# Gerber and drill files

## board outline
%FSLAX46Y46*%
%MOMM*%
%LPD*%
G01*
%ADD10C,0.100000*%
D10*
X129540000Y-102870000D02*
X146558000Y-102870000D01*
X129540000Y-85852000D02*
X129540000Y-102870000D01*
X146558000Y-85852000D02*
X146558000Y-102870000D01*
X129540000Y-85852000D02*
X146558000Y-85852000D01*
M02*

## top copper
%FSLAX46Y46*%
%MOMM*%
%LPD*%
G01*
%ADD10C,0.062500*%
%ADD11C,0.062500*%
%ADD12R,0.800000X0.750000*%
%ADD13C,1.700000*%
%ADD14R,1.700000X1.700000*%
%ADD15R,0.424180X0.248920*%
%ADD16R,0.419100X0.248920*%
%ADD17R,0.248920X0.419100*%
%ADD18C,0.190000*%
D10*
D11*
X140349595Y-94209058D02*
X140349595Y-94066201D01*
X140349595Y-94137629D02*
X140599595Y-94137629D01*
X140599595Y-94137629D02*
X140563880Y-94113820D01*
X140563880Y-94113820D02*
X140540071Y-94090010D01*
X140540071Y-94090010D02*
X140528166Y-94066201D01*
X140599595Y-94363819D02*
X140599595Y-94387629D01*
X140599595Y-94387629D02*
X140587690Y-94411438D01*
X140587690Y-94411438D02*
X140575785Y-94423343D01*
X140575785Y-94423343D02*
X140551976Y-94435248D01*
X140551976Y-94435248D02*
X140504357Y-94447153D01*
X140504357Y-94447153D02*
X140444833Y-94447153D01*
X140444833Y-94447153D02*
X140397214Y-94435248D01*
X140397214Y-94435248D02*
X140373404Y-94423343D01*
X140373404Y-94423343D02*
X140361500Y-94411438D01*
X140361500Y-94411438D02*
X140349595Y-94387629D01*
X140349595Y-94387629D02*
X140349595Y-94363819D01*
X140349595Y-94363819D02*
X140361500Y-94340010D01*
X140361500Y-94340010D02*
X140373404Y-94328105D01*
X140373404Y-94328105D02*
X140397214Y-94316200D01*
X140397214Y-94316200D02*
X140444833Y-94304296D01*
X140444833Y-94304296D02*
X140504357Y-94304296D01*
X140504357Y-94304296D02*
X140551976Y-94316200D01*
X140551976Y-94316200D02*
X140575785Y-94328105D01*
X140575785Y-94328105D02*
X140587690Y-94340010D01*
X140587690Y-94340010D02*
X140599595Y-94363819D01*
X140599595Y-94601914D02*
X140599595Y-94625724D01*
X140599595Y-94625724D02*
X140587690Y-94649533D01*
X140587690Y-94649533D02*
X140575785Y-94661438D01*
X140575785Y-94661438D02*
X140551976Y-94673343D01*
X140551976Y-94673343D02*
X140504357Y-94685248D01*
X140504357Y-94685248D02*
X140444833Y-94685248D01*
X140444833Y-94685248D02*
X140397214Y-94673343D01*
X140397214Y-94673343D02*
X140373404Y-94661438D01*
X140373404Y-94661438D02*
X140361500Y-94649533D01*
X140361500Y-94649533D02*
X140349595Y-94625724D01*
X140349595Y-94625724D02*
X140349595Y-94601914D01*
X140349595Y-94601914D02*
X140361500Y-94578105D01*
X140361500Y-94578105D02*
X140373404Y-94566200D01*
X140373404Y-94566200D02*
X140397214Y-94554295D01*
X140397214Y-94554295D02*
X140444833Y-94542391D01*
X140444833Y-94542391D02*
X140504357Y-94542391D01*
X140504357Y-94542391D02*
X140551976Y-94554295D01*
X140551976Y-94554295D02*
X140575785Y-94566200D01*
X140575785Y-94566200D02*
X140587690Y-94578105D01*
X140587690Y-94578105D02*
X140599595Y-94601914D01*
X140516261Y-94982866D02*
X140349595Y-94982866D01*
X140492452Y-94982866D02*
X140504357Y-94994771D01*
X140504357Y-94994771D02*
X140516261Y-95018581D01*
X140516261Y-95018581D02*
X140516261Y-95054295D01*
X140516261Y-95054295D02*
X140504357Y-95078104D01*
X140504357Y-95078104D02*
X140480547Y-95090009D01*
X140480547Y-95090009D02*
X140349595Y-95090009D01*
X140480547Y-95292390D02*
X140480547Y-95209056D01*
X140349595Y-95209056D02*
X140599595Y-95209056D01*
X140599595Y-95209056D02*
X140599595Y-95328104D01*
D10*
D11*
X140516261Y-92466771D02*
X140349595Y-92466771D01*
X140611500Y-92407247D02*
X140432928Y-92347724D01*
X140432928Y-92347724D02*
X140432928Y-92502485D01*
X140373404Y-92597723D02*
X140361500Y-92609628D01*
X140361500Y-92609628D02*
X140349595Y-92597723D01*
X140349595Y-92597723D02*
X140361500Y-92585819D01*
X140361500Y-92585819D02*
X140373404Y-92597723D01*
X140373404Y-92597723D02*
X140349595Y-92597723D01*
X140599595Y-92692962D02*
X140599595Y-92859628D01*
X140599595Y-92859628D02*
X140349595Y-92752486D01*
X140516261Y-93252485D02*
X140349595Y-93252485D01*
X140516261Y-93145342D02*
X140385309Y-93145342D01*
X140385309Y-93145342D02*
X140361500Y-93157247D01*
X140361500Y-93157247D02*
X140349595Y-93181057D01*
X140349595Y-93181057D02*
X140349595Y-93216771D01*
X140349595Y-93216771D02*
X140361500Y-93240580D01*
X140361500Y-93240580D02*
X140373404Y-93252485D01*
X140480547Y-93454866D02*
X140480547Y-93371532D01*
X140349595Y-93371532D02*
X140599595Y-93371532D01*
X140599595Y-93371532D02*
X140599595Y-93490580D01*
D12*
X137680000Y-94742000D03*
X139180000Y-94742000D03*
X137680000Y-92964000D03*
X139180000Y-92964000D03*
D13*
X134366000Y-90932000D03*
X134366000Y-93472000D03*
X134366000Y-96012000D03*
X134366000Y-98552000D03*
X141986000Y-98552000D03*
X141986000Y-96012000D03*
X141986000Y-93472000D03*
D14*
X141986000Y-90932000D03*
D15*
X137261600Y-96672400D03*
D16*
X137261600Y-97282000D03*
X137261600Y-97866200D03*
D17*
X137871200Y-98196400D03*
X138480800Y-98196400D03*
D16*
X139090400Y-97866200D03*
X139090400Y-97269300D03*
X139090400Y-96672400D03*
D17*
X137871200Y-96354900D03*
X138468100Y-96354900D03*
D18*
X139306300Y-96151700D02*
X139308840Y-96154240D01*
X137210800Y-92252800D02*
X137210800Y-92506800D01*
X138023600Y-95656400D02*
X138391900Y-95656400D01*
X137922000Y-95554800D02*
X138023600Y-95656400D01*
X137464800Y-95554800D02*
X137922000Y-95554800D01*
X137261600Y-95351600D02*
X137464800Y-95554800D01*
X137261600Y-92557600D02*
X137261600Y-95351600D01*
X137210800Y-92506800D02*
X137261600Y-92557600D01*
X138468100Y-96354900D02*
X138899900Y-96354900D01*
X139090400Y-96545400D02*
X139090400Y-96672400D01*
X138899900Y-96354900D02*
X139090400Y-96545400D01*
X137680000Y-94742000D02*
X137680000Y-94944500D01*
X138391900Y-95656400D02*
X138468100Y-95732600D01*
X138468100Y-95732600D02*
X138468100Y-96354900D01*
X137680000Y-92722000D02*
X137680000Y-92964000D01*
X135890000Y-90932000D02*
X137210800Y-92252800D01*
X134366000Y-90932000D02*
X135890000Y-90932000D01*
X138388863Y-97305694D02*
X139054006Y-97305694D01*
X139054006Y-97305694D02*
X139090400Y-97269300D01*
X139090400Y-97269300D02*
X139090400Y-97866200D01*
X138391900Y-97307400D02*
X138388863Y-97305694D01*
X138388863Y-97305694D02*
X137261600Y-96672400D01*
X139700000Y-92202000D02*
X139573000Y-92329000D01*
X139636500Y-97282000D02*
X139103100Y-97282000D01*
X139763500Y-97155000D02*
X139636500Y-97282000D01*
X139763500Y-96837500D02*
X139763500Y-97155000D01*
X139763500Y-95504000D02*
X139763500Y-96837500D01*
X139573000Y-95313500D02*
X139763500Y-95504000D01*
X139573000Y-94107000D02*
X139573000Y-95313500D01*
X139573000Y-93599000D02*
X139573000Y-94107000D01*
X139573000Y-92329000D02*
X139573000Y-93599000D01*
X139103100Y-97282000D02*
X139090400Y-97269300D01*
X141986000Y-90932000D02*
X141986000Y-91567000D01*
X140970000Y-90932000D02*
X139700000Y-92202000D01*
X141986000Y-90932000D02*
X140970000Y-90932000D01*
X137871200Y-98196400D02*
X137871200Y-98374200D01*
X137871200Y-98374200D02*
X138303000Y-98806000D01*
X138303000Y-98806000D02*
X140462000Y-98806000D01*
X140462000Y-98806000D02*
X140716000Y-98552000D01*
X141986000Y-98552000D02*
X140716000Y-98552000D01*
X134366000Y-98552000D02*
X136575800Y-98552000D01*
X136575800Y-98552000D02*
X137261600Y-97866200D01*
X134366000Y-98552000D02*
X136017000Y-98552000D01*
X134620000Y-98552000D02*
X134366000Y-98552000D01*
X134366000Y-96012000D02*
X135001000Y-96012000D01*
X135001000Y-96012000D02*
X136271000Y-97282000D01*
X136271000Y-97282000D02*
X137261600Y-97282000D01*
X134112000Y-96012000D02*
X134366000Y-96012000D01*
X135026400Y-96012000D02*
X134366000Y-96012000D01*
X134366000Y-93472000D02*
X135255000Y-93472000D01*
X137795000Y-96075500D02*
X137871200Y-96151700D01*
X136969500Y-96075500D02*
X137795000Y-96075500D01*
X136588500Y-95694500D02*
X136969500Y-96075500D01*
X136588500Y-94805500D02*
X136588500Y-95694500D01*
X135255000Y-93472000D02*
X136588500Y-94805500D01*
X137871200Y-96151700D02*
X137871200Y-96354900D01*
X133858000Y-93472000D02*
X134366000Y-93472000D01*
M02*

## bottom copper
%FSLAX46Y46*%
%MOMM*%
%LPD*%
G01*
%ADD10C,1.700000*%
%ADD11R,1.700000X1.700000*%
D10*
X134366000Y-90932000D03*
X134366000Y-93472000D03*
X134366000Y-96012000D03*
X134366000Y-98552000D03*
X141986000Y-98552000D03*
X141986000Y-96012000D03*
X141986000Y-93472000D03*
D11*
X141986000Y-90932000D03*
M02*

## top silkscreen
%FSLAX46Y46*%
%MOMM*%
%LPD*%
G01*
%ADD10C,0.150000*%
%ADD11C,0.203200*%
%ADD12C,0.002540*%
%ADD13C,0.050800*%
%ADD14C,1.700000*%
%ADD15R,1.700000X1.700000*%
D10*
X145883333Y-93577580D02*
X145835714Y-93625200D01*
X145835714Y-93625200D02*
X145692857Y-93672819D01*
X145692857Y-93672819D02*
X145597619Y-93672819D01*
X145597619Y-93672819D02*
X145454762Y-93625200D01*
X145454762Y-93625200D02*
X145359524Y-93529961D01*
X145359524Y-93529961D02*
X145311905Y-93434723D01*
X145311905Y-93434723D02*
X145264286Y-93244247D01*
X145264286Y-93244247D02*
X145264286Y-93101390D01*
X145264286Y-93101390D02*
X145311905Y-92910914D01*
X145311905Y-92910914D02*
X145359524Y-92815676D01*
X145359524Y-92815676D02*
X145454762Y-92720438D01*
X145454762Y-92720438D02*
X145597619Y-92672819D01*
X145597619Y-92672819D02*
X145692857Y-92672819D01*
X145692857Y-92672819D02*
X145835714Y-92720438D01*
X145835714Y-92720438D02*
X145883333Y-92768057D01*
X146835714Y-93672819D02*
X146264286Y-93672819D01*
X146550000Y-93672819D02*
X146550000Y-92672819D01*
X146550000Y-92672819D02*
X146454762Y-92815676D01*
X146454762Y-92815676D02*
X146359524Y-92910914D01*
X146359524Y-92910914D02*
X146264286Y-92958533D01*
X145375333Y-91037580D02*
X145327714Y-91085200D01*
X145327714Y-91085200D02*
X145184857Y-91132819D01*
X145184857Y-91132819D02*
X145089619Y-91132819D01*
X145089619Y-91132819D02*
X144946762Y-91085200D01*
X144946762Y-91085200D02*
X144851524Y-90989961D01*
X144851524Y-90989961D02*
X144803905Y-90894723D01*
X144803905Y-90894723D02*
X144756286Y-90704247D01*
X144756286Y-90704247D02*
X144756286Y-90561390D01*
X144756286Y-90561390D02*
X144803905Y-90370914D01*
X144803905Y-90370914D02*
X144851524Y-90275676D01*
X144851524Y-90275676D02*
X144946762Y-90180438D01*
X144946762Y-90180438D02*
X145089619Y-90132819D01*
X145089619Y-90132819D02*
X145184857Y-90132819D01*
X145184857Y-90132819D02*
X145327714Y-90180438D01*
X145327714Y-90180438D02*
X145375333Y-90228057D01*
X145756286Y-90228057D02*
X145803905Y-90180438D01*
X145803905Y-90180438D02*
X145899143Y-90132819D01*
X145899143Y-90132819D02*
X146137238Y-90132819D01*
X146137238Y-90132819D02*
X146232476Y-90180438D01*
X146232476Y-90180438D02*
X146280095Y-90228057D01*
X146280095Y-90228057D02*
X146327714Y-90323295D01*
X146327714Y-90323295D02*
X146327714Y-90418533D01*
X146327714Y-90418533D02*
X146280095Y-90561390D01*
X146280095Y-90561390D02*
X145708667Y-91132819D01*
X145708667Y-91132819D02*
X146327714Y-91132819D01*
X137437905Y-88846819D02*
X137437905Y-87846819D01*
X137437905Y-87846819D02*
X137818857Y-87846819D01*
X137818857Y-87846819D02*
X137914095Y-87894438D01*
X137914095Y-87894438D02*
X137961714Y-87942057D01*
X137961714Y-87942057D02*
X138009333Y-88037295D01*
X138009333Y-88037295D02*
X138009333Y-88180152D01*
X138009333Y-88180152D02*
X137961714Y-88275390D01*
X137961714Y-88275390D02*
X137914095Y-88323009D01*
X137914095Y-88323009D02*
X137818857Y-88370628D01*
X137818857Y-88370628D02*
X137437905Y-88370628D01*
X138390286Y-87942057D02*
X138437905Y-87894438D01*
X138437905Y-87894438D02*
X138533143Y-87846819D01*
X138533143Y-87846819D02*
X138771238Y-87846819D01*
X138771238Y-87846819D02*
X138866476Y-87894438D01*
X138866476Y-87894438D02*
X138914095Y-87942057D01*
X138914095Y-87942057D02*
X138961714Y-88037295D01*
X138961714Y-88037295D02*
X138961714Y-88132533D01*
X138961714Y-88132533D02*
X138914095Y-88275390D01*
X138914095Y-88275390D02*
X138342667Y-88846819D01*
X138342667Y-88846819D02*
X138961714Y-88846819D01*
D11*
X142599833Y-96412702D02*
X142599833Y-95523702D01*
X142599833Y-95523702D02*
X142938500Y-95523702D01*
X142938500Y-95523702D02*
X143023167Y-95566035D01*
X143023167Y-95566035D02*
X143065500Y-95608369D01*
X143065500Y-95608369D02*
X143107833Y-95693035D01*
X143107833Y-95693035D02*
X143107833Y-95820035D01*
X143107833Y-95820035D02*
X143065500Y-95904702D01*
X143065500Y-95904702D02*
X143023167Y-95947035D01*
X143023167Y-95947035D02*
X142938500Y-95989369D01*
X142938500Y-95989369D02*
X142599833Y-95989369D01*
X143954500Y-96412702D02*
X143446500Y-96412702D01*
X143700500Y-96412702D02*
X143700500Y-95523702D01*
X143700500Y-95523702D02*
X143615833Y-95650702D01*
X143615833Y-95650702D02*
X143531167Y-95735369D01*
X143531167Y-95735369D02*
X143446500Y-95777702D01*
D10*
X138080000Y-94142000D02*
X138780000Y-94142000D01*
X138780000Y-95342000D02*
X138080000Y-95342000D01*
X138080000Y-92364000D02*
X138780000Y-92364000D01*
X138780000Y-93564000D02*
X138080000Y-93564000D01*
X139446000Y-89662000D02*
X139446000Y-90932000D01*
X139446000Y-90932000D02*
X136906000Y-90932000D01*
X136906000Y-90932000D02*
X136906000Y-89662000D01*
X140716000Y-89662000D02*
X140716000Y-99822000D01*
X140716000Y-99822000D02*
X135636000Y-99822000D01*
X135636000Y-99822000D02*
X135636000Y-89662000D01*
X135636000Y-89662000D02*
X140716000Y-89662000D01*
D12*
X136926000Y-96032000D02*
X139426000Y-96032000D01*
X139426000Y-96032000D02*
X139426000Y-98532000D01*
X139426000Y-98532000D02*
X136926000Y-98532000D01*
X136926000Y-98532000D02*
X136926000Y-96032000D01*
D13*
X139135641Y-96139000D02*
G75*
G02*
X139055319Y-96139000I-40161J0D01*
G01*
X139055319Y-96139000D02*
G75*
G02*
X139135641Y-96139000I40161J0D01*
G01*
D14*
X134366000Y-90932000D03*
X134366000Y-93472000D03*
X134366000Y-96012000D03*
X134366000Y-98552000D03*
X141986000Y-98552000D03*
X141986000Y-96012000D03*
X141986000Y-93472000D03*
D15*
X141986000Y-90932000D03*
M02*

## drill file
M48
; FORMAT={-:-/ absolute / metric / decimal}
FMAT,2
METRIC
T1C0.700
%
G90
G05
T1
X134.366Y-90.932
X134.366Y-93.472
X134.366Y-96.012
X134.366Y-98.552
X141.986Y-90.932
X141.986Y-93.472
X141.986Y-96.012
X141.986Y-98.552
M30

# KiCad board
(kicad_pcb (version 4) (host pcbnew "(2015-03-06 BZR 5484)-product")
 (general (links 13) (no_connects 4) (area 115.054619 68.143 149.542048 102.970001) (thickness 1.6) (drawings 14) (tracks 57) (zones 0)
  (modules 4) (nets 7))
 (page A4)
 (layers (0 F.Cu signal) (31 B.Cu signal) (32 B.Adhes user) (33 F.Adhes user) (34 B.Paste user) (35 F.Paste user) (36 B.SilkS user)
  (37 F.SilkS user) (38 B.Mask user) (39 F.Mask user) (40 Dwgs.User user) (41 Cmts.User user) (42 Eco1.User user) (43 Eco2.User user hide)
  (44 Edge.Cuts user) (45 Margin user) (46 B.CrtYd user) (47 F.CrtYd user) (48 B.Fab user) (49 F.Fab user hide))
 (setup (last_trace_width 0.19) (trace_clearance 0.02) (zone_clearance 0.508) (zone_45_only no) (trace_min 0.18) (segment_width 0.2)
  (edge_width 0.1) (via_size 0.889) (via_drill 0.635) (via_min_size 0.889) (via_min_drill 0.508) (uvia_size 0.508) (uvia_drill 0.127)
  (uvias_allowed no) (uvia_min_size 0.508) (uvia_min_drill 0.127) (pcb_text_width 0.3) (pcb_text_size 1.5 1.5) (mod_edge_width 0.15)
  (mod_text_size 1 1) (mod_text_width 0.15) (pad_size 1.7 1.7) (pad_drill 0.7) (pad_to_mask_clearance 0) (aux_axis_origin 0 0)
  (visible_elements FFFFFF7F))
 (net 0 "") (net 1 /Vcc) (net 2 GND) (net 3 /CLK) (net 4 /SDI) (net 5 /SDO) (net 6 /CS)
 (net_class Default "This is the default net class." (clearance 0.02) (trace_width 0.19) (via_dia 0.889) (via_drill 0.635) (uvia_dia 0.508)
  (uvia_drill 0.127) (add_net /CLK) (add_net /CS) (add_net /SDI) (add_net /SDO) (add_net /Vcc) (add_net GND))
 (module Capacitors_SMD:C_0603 (layer F.Cu) (at 138.43 94.742)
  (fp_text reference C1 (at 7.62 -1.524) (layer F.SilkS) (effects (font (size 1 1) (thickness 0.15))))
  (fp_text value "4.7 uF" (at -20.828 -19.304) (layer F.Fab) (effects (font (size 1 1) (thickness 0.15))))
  (fp_line (start -0.35 -0.6) (end 0.35 -0.6) (layer F.SilkS) (width 0.15))
  (fp_line (start 0.35 0.6) (end -0.35 0.6) (layer F.SilkS) (width 0.15))
  (pad 1 smd rect (at -0.75 0) (size 0.8 0.75) (layers F.Cu F.Paste F.Mask) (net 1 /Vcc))
  (pad 2 smd rect (at 0.75 0) (size 0.8 0.75) (layers F.Cu F.Paste F.Mask) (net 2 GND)))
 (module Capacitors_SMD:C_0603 (layer F.Cu) (at 138.43 92.964)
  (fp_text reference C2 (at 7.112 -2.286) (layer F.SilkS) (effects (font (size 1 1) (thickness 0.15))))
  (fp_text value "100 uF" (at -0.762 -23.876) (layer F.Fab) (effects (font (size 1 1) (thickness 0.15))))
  (fp_line (start -0.35 -0.6) (end 0.35 -0.6) (layer F.SilkS) (width 0.15))
  (fp_line (start 0.35 0.6) (end -0.35 0.6) (layer F.SilkS) (width 0.15))
  (pad 1 smd rect (at -0.75 0) (size 0.8 0.75) (layers F.Cu F.Paste F.Mask) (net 1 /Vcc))
  (pad 2 smd rect (at 0.75 0) (size 0.8 0.75) (layers F.Cu F.Paste F.Mask) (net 2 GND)))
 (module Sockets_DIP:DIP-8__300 (layer F.Cu) (at 138.176 94.742 270)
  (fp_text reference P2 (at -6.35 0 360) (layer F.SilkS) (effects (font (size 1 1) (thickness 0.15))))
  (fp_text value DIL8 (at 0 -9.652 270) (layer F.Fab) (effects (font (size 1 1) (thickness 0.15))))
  (fp_line (start -5.08 -1.27) (end -3.81 -1.27) (layer F.SilkS) (width 0.15))
  (fp_line (start -3.81 -1.27) (end -3.81 1.27) (layer F.SilkS) (width 0.15))
  (fp_line (start -3.81 1.27) (end -5.08 1.27) (layer F.SilkS) (width 0.15))
  (fp_line (start -5.08 -2.54) (end 5.08 -2.54) (layer F.SilkS) (width 0.15))
  (fp_line (start 5.08 -2.54) (end 5.08 2.54) (layer F.SilkS) (width 0.15))
  (fp_line (start 5.08 2.54) (end -5.08 2.54) (layer F.SilkS) (width 0.15))
  (fp_line (start -5.08 2.54) (end -5.08 -2.54) (layer F.SilkS) (width 0.15))
  (pad 1 thru_hole circle (at -3.81 3.81 270) (size 1.7 1.7) (drill 0.7) (layers *.Cu *.Mask F.SilkS) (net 1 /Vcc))
  (pad 2 thru_hole circle (at -1.27 3.81 270) (size 1.7 1.7) (drill 0.7) (layers *.Cu *.Mask F.SilkS) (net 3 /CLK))
  (pad 3 thru_hole circle (at 1.27 3.81 270) (size 1.7 1.7) (drill 0.7) (layers *.Cu *.Mask F.SilkS) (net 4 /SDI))
  (pad 4 thru_hole circle (at 3.81 3.81 270) (size 1.7 1.7) (drill 0.7) (layers *.Cu *.Mask F.SilkS) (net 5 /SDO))
  (pad 5 thru_hole circle (at 3.81 -3.81 270) (size 1.7 1.7) (drill 0.7) (layers *.Cu *.Mask F.SilkS) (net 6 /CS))
  (pad 6 thru_hole circle (at 1.27 -3.81 270) (size 1.7 1.7) (drill 0.7) (layers *.Cu *.Mask F.SilkS))
  (pad 7 thru_hole circle (at -1.27 -3.81 270) (size 1.7 1.7) (drill 0.7) (layers *.Cu *.Mask F.SilkS))
  (pad 8 thru_hole rect (at -3.81 -3.81 270) (size 1.7 1.7) (drill 0.7) (layers *.Cu *.Mask F.SilkS) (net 2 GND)))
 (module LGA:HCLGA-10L (layer F.Cu) (at 138.176 97.282)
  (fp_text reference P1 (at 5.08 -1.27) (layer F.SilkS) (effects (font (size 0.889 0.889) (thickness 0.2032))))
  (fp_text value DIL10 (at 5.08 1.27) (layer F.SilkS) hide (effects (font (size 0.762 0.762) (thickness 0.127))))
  (fp_line (start -1.25 -1.25) (end 1.25 -1.25) (layer F.SilkS) (width 0.00254))
  (fp_line (start 1.25 -1.25) (end 1.25 1.25) (layer F.SilkS) (width 0.00254))
  (fp_line (start 1.25 1.25) (end -1.25 1.25) (layer F.SilkS) (width 0.00254))
  (fp_line (start -1.25 1.25) (end -1.25 -1.25) (layer F.SilkS) (width 0.00254))
  (fp_circle (center 0.91948 -1.143) (end 0.95758 -1.1303) (layer F.SilkS) (width 0.0508))
  (pad 3 smd rect (at -0.9144 -0.6096) (size 0.42418 0.24892) (layers F.Cu F.Paste F.Mask) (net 2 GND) (clearance 0.05))
  (pad 4 smd rect (at -0.9144 0) (size 0.4191 0.24892) (layers F.Cu F.Paste F.Mask) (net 4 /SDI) (clearance 0.01))
  (pad 5 smd rect (at -0.9144 0.5842) (size 0.4191 0.24892) (layers F.Cu F.Paste F.Mask) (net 5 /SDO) (clearance 0.01))
  (pad 6 smd rect (at -0.3048 0.9144) (size 0.24892 0.4191) (layers F.Cu F.Paste F.Mask) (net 6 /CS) (clearance 0.05))
  (pad 7 smd rect (at 0.3048 0.9144) (size 0.24892 0.4191) (layers F.Cu F.Paste F.Mask) (clearance 0.05))
  (pad 8 smd rect (at 0.9144 0.5842) (size 0.4191 0.24892) (layers F.Cu F.Paste F.Mask) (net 2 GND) (clearance 0.05))
  (pad 9 smd rect (at 0.9144 -0.0127) (size 0.4191 0.24892) (layers F.Cu F.Paste F.Mask) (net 2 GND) (clearance 0.05))
  (pad 10 smd rect (at 0.9144 -0.6096) (size 0.4191 0.24892) (layers F.Cu F.Paste F.Mask) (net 1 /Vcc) (clearance 0.05))
  (pad 2 smd rect (at -0.3048 -0.9271) (size 0.24892 0.4191) (layers F.Cu F.Paste F.Mask) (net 3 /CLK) (clearance 0.05))
  (pad 1 smd rect (at 0.2921 -0.9271) (size 0.24892 0.4191) (layers F.Cu F.Paste F.Mask) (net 1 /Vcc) (clearance 0.05)))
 (gr_line (start 129.54 102.87) (end 146.558 102.87) (angle 90) (layer Edge.Cuts) (width 0.1))
 (gr_line (start 129.54 85.852) (end 129.54 102.87) (angle 90) (layer Edge.Cuts) (width 0.1))
 (gr_line (start 146.558 85.852) (end 146.558 102.87) (angle 90) (layer Edge.Cuts) (width 0.1))
 (gr_line (start 129.54 85.852) (end 146.558 85.852) (angle 90) (layer Edge.Cuts) (width 0.1))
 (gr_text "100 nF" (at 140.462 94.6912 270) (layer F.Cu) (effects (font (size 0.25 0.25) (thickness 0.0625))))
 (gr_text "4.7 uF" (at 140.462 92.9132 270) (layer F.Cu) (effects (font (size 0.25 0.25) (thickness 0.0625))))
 (segment (start 139.3063 96.1517) (end 139.30884 96.15424) (width 0.19) (layer F.Cu) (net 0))
 (segment (start 137.2108 92.2528) (end 137.2108 92.5068) (width 0.19) (layer F.Cu) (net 1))
 (segment (start 138.0236 95.6564) (end 138.3919 95.6564) (width 0.19) (layer F.Cu) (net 1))
 (segment (start 137.922 95.5548) (end 138.0236 95.6564) (width 0.19) (layer F.Cu) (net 1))
 (segment (start 137.4648 95.5548) (end 137.922 95.5548) (width 0.19) (layer F.Cu) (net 1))
 (segment (start 137.2616 95.3516) (end 137.4648 95.5548) (width 0.19) (layer F.Cu) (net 1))
 (segment (start 137.2616 92.5576) (end 137.2616 95.3516) (width 0.19) (layer F.Cu) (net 1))
 (segment (start 137.2108 92.5068) (end 137.2616 92.5576) (width 0.19) (layer F.Cu) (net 1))
 (segment (start 138.4681 96.3549) (end 138.8999 96.3549) (width 0.19) (layer F.Cu) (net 1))
 (segment (start 139.0904 96.5454) (end 139.0904 96.6724) (width 0.19) (layer F.Cu) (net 1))
 (segment (start 138.8999 96.3549) (end 139.0904 96.5454) (width 0.19) (layer F.Cu) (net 1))
 (segment (start 137.68 94.742) (end 137.68 94.9445) (width 0.19) (layer F.Cu) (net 1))
 (segment (start 138.3919 95.6564) (end 138.4681 95.7326) (width 0.19) (layer F.Cu) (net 1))
 (segment (start 138.4681 95.7326) (end 138.4681 96.3549) (width 0.19) (layer F.Cu) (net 1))
 (segment (start 137.68 92.722) (end 137.68 92.964) (width 0.19) (layer F.Cu) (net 1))
 (segment (start 135.89 90.932) (end 137.2108 92.2528) (width 0.19) (layer F.Cu) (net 1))
 (segment (start 134.366 90.932) (end 135.89 90.932) (width 0.19) (layer F.Cu) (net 1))
 (segment (start 138.388863 97.305694) (end 139.054006 97.305694) (width 0.19) (layer F.Cu) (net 2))
 (segment (start 139.054006 97.305694) (end 139.0904 97.2693) (width 0.19) (layer F.Cu) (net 2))
 (segment (start 139.0904 97.2693) (end 139.0904 97.8662) (width 0.19) (layer F.Cu) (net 2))
 (segment (start 138.3919 97.3074) (end 138.388863 97.305694) (width 0.19) (layer F.Cu) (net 2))
 (segment (start 138.388863 97.305694) (end 137.2616 96.6724) (width 0.19) (layer F.Cu) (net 2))
 (segment (start 139.7 92.202) (end 139.573 92.329) (width 0.19) (layer F.Cu) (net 2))
 (segment (start 139.6365 97.282) (end 139.1031 97.282) (width 0.19) (layer F.Cu) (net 2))
 (segment (start 139.7635 97.155) (end 139.6365 97.282) (width 0.19) (layer F.Cu) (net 2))
 (segment (start 139.7635 96.8375) (end 139.7635 97.155) (width 0.19) (layer F.Cu) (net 2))
 (segment (start 139.7635 95.504) (end 139.7635 96.8375) (width 0.19) (layer F.Cu) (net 2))
 (segment (start 139.573 95.3135) (end 139.7635 95.504) (width 0.19) (layer F.Cu) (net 2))
 (segment (start 139.573 94.107) (end 139.573 95.3135) (width 0.19) (layer F.Cu) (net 2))
 (segment (start 139.573 93.599) (end 139.573 94.107) (width 0.19) (layer F.Cu) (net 2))
 (segment (start 139.573 92.329) (end 139.573 93.599) (width 0.19) (layer F.Cu) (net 2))
 (segment (start 139.1031 97.282) (end 139.0904 97.2693) (width 0.19) (layer F.Cu) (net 2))
 (segment (start 141.986 90.932) (end 141.986 91.567) (width 0.19) (layer F.Cu) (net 2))
 (segment (start 140.97 90.932) (end 139.7 92.202) (width 0.19) (layer F.Cu) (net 2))
 (segment (start 141.986 90.932) (end 140.97 90.932) (width 0.19) (layer F.Cu) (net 2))
 (segment (start 137.8712 98.1964) (end 137.8712 98.3742) (width 0.19) (layer F.Cu) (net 6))
 (segment (start 137.8712 98.3742) (end 138.303 98.806) (width 0.19) (layer F.Cu) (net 6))
 (segment (start 138.303 98.806) (end 140.462 98.806) (width 0.19) (layer F.Cu) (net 6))
 (segment (start 140.462 98.806) (end 140.716 98.552) (width 0.19) (layer F.Cu) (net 6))
 (segment (start 141.986 98.552) (end 140.716 98.552) (width 0.19) (layer F.Cu) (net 6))
 (segment (start 134.366 98.552) (end 136.5758 98.552) (width 0.19) (layer F.Cu) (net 5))
 (segment (start 136.5758 98.552) (end 137.2616 97.8662) (width 0.19) (layer F.Cu) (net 5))
 (segment (start 134.366 98.552) (end 136.017 98.552) (width 0.19) (layer F.Cu) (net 5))
 (segment (start 134.62 98.552) (end 134.366 98.552) (width 0.19) (layer F.Cu) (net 5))
 (segment (start 134.366 96.012) (end 135.001 96.012) (width 0.19) (layer F.Cu) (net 4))
 (segment (start 135.001 96.012) (end 136.271 97.282) (width 0.19) (layer F.Cu) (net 4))
 (segment (start 136.271 97.282) (end 137.2616 97.282) (width 0.19) (layer F.Cu) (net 4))
 (segment (start 134.112 96.012) (end 134.366 96.012) (width 0.19) (layer F.Cu) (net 4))
 (segment (start 135.0264 96.012) (end 134.366 96.012) (width 0.19) (layer F.Cu) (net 4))
 (segment (start 134.366 93.472) (end 135.255 93.472) (width 0.19) (layer F.Cu) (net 3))
 (segment (start 137.795 96.0755) (end 137.8712 96.1517) (width 0.19) (layer F.Cu) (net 3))
 (segment (start 136.9695 96.0755) (end 137.795 96.0755) (width 0.19) (layer F.Cu) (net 3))
 (segment (start 136.5885 95.6945) (end 136.9695 96.0755) (width 0.19) (layer F.Cu) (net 3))
 (segment (start 136.5885 94.8055) (end 136.5885 95.6945) (width 0.19) (layer F.Cu) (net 3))
 (segment (start 135.255 93.472) (end 136.5885 94.8055) (width 0.19) (layer F.Cu) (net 3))
 (segment (start 137.8712 96.1517) (end 137.8712 96.3549) (width 0.19) (layer F.Cu) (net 3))
 (segment (start 133.858 93.472) (end 134.366 93.472) (width 0.19) (layer F.Cu) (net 3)))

